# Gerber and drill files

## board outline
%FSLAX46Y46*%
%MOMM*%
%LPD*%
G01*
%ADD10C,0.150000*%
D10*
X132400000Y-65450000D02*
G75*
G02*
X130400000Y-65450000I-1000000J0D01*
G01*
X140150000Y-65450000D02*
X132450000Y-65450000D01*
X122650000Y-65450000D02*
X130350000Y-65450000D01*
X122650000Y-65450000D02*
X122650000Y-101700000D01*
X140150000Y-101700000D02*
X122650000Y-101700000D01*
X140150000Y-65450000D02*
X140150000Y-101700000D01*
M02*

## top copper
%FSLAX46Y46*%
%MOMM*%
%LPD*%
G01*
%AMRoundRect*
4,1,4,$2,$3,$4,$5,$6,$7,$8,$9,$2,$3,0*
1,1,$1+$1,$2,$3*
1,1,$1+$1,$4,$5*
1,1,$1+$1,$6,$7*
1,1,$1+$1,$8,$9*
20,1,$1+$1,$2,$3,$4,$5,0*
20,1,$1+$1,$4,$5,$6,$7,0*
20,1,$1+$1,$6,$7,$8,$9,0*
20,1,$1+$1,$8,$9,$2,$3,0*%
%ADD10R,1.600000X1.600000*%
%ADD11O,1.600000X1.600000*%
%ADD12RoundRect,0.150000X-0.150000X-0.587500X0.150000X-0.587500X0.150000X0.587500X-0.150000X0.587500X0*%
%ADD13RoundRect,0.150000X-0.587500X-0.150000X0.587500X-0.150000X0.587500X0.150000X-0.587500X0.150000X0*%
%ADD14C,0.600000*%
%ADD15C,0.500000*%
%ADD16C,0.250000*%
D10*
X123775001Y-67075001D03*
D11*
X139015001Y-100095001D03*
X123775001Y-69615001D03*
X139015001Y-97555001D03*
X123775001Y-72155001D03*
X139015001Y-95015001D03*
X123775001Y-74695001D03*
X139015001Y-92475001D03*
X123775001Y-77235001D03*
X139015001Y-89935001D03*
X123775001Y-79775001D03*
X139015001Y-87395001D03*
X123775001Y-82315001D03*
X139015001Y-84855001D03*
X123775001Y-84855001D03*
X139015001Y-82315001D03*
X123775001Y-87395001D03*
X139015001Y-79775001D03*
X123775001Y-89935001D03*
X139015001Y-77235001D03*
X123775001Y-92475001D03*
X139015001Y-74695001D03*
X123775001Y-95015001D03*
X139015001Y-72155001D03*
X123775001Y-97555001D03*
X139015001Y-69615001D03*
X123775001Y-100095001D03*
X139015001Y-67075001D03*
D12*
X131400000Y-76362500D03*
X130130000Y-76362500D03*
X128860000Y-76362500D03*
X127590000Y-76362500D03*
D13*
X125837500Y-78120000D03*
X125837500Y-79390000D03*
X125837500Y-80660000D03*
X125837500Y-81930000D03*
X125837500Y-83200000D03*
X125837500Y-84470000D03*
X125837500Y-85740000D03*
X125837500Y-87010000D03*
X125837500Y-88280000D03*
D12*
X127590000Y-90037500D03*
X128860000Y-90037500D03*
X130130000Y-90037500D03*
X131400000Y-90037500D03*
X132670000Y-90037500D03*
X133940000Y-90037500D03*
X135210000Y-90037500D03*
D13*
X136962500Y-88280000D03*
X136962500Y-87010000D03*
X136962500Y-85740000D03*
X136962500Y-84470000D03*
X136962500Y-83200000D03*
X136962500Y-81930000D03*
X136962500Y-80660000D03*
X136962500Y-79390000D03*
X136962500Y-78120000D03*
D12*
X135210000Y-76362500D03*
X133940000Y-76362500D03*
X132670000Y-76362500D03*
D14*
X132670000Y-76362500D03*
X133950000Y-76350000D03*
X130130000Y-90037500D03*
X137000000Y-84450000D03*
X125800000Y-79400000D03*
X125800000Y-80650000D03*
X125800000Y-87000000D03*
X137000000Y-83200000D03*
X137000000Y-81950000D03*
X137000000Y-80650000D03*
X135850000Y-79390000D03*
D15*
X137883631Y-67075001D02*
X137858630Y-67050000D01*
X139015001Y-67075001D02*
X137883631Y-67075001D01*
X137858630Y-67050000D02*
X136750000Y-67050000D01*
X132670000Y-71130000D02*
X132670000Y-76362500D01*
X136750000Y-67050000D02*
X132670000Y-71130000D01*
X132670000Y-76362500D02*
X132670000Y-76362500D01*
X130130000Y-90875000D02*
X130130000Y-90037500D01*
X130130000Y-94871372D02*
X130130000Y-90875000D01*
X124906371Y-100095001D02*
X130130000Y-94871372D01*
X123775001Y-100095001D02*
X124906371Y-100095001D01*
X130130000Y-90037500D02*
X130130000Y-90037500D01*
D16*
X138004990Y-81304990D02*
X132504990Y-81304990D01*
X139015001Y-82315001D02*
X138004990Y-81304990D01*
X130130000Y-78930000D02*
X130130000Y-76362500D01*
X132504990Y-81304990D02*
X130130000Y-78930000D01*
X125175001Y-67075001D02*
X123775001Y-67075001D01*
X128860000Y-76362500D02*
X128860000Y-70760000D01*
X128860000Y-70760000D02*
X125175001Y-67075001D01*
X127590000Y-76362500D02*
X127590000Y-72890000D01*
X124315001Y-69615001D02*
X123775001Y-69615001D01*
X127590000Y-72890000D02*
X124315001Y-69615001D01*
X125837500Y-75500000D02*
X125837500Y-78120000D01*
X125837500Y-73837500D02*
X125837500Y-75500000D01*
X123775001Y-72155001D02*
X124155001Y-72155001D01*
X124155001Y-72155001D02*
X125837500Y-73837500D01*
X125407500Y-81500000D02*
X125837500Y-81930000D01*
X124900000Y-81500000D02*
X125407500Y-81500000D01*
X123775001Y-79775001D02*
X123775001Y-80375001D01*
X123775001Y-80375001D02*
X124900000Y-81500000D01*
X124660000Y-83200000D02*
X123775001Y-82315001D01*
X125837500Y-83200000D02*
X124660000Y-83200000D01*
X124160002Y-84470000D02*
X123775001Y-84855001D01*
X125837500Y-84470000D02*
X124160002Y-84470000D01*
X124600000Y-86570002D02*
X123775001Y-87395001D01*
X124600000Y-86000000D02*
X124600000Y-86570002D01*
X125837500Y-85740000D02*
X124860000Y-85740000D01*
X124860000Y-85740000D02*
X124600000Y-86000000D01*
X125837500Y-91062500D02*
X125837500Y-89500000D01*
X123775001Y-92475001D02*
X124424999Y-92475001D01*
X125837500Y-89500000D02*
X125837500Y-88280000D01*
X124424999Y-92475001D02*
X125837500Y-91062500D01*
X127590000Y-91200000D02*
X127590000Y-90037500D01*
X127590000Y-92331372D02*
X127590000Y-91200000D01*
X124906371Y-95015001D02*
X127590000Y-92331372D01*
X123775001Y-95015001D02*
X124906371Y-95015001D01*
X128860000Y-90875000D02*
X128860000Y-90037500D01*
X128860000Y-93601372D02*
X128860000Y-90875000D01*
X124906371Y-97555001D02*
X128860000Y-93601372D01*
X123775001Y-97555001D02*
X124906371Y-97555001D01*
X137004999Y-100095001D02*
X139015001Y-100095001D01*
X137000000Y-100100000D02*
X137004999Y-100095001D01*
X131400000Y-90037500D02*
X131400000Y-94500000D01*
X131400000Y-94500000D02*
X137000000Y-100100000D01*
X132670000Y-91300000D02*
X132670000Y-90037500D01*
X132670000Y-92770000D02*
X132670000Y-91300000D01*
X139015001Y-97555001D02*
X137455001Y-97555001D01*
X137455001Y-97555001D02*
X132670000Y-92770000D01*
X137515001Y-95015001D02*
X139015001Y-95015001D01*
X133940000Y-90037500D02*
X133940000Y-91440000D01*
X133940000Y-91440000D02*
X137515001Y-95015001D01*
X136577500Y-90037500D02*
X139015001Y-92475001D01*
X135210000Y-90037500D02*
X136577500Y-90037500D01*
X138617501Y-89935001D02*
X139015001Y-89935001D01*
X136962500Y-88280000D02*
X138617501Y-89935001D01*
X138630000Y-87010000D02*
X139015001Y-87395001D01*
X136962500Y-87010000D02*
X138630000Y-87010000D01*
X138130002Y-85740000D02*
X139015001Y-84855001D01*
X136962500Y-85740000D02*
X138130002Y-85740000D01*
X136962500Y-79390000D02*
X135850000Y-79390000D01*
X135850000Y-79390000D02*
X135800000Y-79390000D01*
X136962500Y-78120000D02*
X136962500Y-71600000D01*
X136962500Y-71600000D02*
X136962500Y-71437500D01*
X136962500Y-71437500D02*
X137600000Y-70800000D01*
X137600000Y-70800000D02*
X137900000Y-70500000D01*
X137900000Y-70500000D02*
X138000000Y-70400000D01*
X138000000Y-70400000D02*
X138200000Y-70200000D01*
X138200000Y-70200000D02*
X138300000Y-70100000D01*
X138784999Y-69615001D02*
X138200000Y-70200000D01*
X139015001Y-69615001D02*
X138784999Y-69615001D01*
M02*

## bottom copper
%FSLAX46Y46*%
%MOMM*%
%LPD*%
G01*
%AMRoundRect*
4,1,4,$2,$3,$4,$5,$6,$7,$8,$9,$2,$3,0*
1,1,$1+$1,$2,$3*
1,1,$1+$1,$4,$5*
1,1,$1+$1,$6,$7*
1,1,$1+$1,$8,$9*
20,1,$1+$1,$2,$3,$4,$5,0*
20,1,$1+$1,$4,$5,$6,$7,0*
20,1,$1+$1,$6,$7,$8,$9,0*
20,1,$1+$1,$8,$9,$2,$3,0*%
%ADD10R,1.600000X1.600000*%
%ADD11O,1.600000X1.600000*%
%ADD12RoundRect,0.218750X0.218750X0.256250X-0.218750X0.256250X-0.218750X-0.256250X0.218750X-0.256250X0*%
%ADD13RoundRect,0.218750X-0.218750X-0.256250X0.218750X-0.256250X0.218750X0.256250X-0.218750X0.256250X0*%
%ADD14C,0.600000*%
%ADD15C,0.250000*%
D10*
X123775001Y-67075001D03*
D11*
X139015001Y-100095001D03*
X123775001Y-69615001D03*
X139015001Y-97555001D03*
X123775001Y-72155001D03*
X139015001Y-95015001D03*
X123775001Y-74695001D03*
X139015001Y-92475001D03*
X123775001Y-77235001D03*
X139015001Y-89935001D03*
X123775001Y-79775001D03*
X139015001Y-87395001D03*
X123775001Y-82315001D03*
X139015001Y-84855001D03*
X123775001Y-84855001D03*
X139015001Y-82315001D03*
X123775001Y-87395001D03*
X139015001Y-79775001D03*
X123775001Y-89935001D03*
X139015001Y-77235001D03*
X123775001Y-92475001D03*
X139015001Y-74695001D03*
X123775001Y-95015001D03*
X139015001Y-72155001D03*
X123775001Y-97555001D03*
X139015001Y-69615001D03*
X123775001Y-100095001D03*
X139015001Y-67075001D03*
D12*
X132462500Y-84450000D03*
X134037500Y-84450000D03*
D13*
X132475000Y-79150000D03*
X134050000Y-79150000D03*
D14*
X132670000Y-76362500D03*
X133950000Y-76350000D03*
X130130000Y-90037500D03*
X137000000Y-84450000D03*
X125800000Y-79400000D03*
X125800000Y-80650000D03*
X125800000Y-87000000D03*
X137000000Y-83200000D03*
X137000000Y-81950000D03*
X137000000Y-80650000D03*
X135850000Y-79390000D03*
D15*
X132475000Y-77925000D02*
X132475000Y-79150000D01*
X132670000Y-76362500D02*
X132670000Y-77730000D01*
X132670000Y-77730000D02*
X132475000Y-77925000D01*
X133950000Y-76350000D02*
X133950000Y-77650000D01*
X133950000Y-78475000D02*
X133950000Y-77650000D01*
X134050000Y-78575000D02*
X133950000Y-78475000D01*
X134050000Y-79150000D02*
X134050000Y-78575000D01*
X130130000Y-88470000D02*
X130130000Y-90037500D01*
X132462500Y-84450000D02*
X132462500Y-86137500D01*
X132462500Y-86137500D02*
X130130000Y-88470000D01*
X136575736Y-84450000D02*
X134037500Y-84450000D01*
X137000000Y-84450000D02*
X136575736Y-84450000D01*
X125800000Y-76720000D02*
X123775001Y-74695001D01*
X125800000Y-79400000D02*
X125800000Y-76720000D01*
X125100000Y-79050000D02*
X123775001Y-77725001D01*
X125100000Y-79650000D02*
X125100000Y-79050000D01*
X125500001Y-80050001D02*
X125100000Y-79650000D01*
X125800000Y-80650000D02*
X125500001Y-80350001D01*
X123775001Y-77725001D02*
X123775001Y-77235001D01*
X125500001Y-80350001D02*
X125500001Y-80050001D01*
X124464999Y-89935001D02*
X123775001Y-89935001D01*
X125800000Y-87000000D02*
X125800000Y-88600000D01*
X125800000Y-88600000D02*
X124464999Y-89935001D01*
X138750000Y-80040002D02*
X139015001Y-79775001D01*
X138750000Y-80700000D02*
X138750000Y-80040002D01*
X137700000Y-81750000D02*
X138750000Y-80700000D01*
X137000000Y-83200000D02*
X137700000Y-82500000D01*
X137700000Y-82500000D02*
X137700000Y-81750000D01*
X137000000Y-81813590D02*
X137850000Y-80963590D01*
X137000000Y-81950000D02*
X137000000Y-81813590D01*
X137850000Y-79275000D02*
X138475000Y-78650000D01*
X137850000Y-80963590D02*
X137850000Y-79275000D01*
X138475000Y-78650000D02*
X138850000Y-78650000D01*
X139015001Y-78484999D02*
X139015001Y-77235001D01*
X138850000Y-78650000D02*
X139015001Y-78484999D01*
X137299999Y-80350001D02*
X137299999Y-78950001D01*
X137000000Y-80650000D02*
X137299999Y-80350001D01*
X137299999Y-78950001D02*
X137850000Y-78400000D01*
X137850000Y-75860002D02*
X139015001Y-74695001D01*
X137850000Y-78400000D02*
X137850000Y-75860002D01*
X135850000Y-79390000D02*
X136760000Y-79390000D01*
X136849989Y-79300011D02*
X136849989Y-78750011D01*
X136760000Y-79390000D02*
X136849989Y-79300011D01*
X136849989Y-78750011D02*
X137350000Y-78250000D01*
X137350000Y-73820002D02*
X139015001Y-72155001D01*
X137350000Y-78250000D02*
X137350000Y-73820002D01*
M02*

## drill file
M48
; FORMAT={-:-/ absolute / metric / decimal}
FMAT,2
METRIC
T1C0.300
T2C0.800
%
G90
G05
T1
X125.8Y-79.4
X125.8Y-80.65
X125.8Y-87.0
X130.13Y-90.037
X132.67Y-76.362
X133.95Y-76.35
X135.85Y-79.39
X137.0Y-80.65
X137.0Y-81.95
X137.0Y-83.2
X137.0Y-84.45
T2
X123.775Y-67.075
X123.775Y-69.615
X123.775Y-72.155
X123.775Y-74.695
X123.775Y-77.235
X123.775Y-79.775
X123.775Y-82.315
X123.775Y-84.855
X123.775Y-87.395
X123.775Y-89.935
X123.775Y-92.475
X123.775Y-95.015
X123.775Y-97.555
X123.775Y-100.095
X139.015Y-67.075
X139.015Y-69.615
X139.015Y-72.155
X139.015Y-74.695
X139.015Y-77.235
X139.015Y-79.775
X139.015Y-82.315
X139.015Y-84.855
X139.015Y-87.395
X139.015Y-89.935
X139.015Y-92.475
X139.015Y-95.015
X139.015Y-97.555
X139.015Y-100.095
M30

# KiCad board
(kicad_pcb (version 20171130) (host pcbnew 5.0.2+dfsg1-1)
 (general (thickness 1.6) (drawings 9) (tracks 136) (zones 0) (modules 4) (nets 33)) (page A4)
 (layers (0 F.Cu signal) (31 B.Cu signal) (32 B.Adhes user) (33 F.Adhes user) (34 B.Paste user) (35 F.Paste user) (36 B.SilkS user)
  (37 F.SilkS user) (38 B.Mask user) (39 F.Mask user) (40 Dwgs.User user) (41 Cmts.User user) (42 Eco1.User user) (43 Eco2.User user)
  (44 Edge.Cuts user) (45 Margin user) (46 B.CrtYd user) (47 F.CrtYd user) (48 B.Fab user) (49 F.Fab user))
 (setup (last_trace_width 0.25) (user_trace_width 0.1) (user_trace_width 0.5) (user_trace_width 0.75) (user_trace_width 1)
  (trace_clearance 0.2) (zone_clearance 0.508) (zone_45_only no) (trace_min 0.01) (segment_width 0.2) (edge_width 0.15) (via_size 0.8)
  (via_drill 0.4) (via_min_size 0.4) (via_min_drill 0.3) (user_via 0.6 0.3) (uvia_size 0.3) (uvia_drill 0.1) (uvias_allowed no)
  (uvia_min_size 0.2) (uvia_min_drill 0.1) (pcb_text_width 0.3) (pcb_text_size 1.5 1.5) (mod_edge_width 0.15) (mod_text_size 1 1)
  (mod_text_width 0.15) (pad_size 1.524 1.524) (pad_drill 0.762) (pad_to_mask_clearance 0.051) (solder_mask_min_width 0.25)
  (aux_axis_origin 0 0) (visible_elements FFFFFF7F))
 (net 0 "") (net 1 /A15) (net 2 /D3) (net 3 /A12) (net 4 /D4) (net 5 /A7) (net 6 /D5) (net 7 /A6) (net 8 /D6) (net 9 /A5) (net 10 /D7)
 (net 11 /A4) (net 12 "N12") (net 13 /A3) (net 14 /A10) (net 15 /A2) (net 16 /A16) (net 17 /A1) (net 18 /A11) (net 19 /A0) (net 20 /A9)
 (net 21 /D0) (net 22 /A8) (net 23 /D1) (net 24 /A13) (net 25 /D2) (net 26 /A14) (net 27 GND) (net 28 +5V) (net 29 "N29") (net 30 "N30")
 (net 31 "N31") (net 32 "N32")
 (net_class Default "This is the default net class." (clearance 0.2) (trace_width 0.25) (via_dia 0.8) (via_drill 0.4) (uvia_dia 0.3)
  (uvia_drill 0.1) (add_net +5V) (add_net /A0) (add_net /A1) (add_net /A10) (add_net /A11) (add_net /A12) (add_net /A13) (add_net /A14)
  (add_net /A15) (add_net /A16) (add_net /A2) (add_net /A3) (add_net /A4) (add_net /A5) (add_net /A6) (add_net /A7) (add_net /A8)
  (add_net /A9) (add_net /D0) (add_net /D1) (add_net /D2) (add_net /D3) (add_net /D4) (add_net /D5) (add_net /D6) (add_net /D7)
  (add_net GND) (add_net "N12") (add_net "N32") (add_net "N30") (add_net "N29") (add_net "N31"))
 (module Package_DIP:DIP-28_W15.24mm (layer F.Cu) (at 123.775001 67.075001)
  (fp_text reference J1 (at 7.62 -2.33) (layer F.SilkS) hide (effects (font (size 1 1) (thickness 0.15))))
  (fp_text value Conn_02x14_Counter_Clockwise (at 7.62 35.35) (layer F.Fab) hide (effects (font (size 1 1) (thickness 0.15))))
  (pad 1 thru_hole rect (at 0 0) (size 1.6 1.6) (drill 0.8) (layers *.Cu *.Mask) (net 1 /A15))
  (pad 15 thru_hole oval (at 15.24 33.02) (size 1.6 1.6) (drill 0.8) (layers *.Cu *.Mask) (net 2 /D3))
  (pad 2 thru_hole oval (at 0 2.54) (size 1.6 1.6) (drill 0.8) (layers *.Cu *.Mask) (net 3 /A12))
  (pad 16 thru_hole oval (at 15.24 30.48) (size 1.6 1.6) (drill 0.8) (layers *.Cu *.Mask) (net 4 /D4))
  (pad 3 thru_hole oval (at 0 5.08) (size 1.6 1.6) (drill 0.8) (layers *.Cu *.Mask) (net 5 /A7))
  (pad 17 thru_hole oval (at 15.24 27.94) (size 1.6 1.6) (drill 0.8) (layers *.Cu *.Mask) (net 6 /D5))
  (pad 4 thru_hole oval (at 0 7.62) (size 1.6 1.6) (drill 0.8) (layers *.Cu *.Mask) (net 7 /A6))
  (pad 18 thru_hole oval (at 15.24 25.4) (size 1.6 1.6) (drill 0.8) (layers *.Cu *.Mask) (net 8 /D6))
  (pad 5 thru_hole oval (at 0 10.16) (size 1.6 1.6) (drill 0.8) (layers *.Cu *.Mask) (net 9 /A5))
  (pad 19 thru_hole oval (at 15.24 22.86) (size 1.6 1.6) (drill 0.8) (layers *.Cu *.Mask) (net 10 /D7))
  (pad 6 thru_hole oval (at 0 12.7) (size 1.6 1.6) (drill 0.8) (layers *.Cu *.Mask) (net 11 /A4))
  (pad 20 thru_hole oval (at 15.24 20.32) (size 1.6 1.6) (drill 0.8) (layers *.Cu *.Mask) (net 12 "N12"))
  (pad 7 thru_hole oval (at 0 15.24) (size 1.6 1.6) (drill 0.8) (layers *.Cu *.Mask) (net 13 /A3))
  (pad 21 thru_hole oval (at 15.24 17.78) (size 1.6 1.6) (drill 0.8) (layers *.Cu *.Mask) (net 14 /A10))
  (pad 8 thru_hole oval (at 0 17.78) (size 1.6 1.6) (drill 0.8) (layers *.Cu *.Mask) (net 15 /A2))
  (pad 22 thru_hole oval (at 15.24 15.24) (size 1.6 1.6) (drill 0.8) (layers *.Cu *.Mask) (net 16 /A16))
  (pad 9 thru_hole oval (at 0 20.32) (size 1.6 1.6) (drill 0.8) (layers *.Cu *.Mask) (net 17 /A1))
  (pad 23 thru_hole oval (at 15.24 12.7) (size 1.6 1.6) (drill 0.8) (layers *.Cu *.Mask) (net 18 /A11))
  (pad 10 thru_hole oval (at 0 22.86) (size 1.6 1.6) (drill 0.8) (layers *.Cu *.Mask) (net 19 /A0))
  (pad 24 thru_hole oval (at 15.24 10.16) (size 1.6 1.6) (drill 0.8) (layers *.Cu *.Mask) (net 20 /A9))
  (pad 11 thru_hole oval (at 0 25.4) (size 1.6 1.6) (drill 0.8) (layers *.Cu *.Mask) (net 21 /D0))
  (pad 25 thru_hole oval (at 15.24 7.62) (size 1.6 1.6) (drill 0.8) (layers *.Cu *.Mask) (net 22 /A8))
  (pad 12 thru_hole oval (at 0 27.94) (size 1.6 1.6) (drill 0.8) (layers *.Cu *.Mask) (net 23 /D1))
  (pad 26 thru_hole oval (at 15.24 5.08) (size 1.6 1.6) (drill 0.8) (layers *.Cu *.Mask) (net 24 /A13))
  (pad 13 thru_hole oval (at 0 30.48) (size 1.6 1.6) (drill 0.8) (layers *.Cu *.Mask) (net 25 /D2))
  (pad 27 thru_hole oval (at 15.24 2.54) (size 1.6 1.6) (drill 0.8) (layers *.Cu *.Mask) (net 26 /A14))
  (pad 14 thru_hole oval (at 0 33.02) (size 1.6 1.6) (drill 0.8) (layers *.Cu *.Mask) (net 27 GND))
  (pad 28 thru_hole oval (at 15.24 0) (size 1.6 1.6) (drill 0.8) (layers *.Cu *.Mask) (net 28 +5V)))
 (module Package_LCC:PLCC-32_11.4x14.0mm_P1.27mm (layer F.Cu) (at 131.4 83.2)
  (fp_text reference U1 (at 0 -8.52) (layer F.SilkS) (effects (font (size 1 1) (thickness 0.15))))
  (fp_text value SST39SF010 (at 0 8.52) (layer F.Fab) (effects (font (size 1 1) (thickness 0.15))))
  (pad 1 smd roundrect (at 0 -6.8375) (size 0.6 1.475) (layers F.Cu F.Paste F.Mask) (roundrect_rratio 0.25) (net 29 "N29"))
  (pad 2 smd roundrect (at -1.27 -6.8375) (size 0.6 1.475) (layers F.Cu F.Paste F.Mask) (roundrect_rratio 0.25) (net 16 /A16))
  (pad 3 smd roundrect (at -2.54 -6.8375) (size 0.6 1.475) (layers F.Cu F.Paste F.Mask) (roundrect_rratio 0.25) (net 1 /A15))
  (pad 4 smd roundrect (at -3.81 -6.8375) (size 0.6 1.475) (layers F.Cu F.Paste F.Mask) (roundrect_rratio 0.25) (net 3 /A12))
  (pad 5 smd roundrect (at -5.5625 -5.08) (size 1.475 0.6) (layers F.Cu F.Paste F.Mask) (roundrect_rratio 0.25) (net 5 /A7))
  (pad 6 smd roundrect (at -5.5625 -3.81) (size 1.475 0.6) (layers F.Cu F.Paste F.Mask) (roundrect_rratio 0.25) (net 7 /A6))
  (pad 7 smd roundrect (at -5.5625 -2.54) (size 1.475 0.6) (layers F.Cu F.Paste F.Mask) (roundrect_rratio 0.25) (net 9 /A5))
  (pad 8 smd roundrect (at -5.5625 -1.27) (size 1.475 0.6) (layers F.Cu F.Paste F.Mask) (roundrect_rratio 0.25) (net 11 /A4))
  (pad 9 smd roundrect (at -5.5625 0) (size 1.475 0.6) (layers F.Cu F.Paste F.Mask) (roundrect_rratio 0.25) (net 13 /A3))
  (pad 10 smd roundrect (at -5.5625 1.27) (size 1.475 0.6) (layers F.Cu F.Paste F.Mask) (roundrect_rratio 0.25) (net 15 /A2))
  (pad 11 smd roundrect (at -5.5625 2.54) (size 1.475 0.6) (layers F.Cu F.Paste F.Mask) (roundrect_rratio 0.25) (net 17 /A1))
  (pad 12 smd roundrect (at -5.5625 3.81) (size 1.475 0.6) (layers F.Cu F.Paste F.Mask) (roundrect_rratio 0.25) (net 19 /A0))
  (pad 13 smd roundrect (at -5.5625 5.08) (size 1.475 0.6) (layers F.Cu F.Paste F.Mask) (roundrect_rratio 0.25) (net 21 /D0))
  (pad 14 smd roundrect (at -3.81 6.8375) (size 0.6 1.475) (layers F.Cu F.Paste F.Mask) (roundrect_rratio 0.25) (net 23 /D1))
  (pad 15 smd roundrect (at -2.54 6.8375) (size 0.6 1.475) (layers F.Cu F.Paste F.Mask) (roundrect_rratio 0.25) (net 25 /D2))
  (pad 16 smd roundrect (at -1.27 6.8375) (size 0.6 1.475) (layers F.Cu F.Paste F.Mask) (roundrect_rratio 0.25) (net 27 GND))
  (pad 17 smd roundrect (at 0 6.8375) (size 0.6 1.475) (layers F.Cu F.Paste F.Mask) (roundrect_rratio 0.25) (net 2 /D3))
  (pad 18 smd roundrect (at 1.27 6.8375) (size 0.6 1.475) (layers F.Cu F.Paste F.Mask) (roundrect_rratio 0.25) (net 4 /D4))
  (pad 19 smd roundrect (at 2.54 6.8375) (size 0.6 1.475) (layers F.Cu F.Paste F.Mask) (roundrect_rratio 0.25) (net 6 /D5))
  (pad 20 smd roundrect (at 3.81 6.8375) (size 0.6 1.475) (layers F.Cu F.Paste F.Mask) (roundrect_rratio 0.25) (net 8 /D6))
  (pad 21 smd roundrect (at 5.5625 5.08) (size 1.475 0.6) (layers F.Cu F.Paste F.Mask) (roundrect_rratio 0.25) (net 10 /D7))
  (pad 22 smd roundrect (at 5.5625 3.81) (size 1.475 0.6) (layers F.Cu F.Paste F.Mask) (roundrect_rratio 0.25) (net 12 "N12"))
  (pad 23 smd roundrect (at 5.5625 2.54) (size 1.475 0.6) (layers F.Cu F.Paste F.Mask) (roundrect_rratio 0.25) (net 14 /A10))
  (pad 24 smd roundrect (at 5.5625 1.27) (size 1.475 0.6) (layers F.Cu F.Paste F.Mask) (roundrect_rratio 0.25) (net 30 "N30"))
  (pad 25 smd roundrect (at 5.5625 0) (size 1.475 0.6) (layers F.Cu F.Paste F.Mask) (roundrect_rratio 0.25) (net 18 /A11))
  (pad 26 smd roundrect (at 5.5625 -1.27) (size 1.475 0.6) (layers F.Cu F.Paste F.Mask) (roundrect_rratio 0.25) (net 20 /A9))
  (pad 27 smd roundrect (at 5.5625 -2.54) (size 1.475 0.6) (layers F.Cu F.Paste F.Mask) (roundrect_rratio 0.25) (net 22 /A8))
  (pad 28 smd roundrect (at 5.5625 -3.81) (size 1.475 0.6) (layers F.Cu F.Paste F.Mask) (roundrect_rratio 0.25) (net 24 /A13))
  (pad 29 smd roundrect (at 5.5625 -5.08) (size 1.475 0.6) (layers F.Cu F.Paste F.Mask) (roundrect_rratio 0.25) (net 26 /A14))
  (pad 30 smd roundrect (at 3.81 -6.8375) (size 0.6 1.475) (layers F.Cu F.Paste F.Mask) (roundrect_rratio 0.25) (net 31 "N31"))
  (pad 31 smd roundrect (at 2.54 -6.8375) (size 0.6 1.475) (layers F.Cu F.Paste F.Mask) (roundrect_rratio 0.25) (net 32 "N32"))
  (pad 32 smd roundrect (at 1.27 -6.8375) (size 0.6 1.475) (layers F.Cu F.Paste F.Mask) (roundrect_rratio 0.25) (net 28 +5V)))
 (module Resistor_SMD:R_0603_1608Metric (layer B.Cu) (at 133.25 84.45 180)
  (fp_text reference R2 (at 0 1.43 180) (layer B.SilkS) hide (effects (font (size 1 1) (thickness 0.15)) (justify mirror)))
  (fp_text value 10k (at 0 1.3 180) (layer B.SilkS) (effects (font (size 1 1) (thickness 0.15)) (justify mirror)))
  (pad 2 smd roundrect (at 0.7875 0 180) (size 0.875 0.95) (layers B.Cu B.Paste B.Mask) (roundrect_rratio 0.25) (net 27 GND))
  (pad 1 smd roundrect (at -0.7875 0 180) (size 0.875 0.95) (layers B.Cu B.Paste B.Mask) (roundrect_rratio 0.25) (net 30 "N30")))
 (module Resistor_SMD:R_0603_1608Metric (layer B.Cu) (at 133.2625 79.15)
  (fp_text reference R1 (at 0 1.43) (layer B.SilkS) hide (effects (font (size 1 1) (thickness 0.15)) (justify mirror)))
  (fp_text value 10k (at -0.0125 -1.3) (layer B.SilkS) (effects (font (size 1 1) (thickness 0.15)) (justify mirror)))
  (pad 1 smd roundrect (at -0.7875 0) (size 0.875 0.95) (layers B.Cu B.Paste B.Mask) (roundrect_rratio 0.25) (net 28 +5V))
  (pad 2 smd roundrect (at 0.7875 0) (size 0.875 0.95) (layers B.Cu B.Paste B.Mask) (roundrect_rratio 0.25) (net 32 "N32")))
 (gr_arc (start 131.4 65.45) (end 130.4 65.45) (angle -180) (layer Edge.Cuts) (width 0.15))
 (gr_line (start 140.15 65.45) (end 132.45 65.45) (layer Edge.Cuts) (width 0.15))
 (gr_line (start 122.65 65.45) (end 130.35 65.45) (layer Edge.Cuts) (width 0.15))
 (gr_line (start 122.65 65.45) (end 122.65 101.7) (layer Edge.Cuts) (width 0.15))
 (gr_line (start 140.15 101.7) (end 122.65 101.7) (layer Edge.Cuts) (width 0.15))
 (gr_line (start 140.15 65.45) (end 140.15 101.7) (layer Edge.Cuts) (width 0.15))
 (segment (start 137.883631 67.075001) (end 137.85863 67.05) (width 0.5) (layer F.Cu) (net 28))
 (segment (start 139.015001 67.075001) (end 137.883631 67.075001) (width 0.5) (layer F.Cu) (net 28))
 (segment (start 137.85863 67.05) (end 136.75 67.05) (width 0.5) (layer F.Cu) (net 28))
 (segment (start 132.67 71.13) (end 132.67 76.3625) (width 0.5) (layer F.Cu) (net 28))
 (segment (start 136.75 67.05) (end 132.67 71.13) (width 0.5) (layer F.Cu) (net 28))
 (segment (start 132.67 76.3625) (end 132.67 76.3625) (width 0.5) (layer F.Cu) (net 28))
 (via (at 132.67 76.3625) (size 0.6) (drill 0.3) (layers F.Cu B.Cu) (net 28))
 (segment (start 132.475 77.925) (end 132.475 79.15) (width 0.25) (layer B.Cu) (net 28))
 (segment (start 132.67 76.3625) (end 132.67 77.73) (width 0.25) (layer B.Cu) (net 28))
 (segment (start 132.67 77.73) (end 132.475 77.925) (width 0.25) (layer B.Cu) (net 28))
 (via (at 133.95 76.35) (size 0.6) (drill 0.3) (layers F.Cu B.Cu) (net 32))
 (segment (start 133.95 76.35) (end 133.95 77.65) (width 0.25) (layer B.Cu) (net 32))
 (segment (start 133.95 78.475) (end 133.95 77.65) (width 0.25) (layer B.Cu) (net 32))
 (segment (start 134.05 78.575) (end 133.95 78.475) (width 0.25) (layer B.Cu) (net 32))
 (segment (start 134.05 79.15) (end 134.05 78.575) (width 0.25) (layer B.Cu) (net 32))
 (segment (start 130.13 90.875) (end 130.13 90.0375) (width 0.5) (layer F.Cu) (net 27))
 (segment (start 130.13 94.871372) (end 130.13 90.875) (width 0.5) (layer F.Cu) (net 27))
 (segment (start 124.906371 100.095001) (end 130.13 94.871372) (width 0.5) (layer F.Cu) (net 27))
 (segment (start 123.775001 100.095001) (end 124.906371 100.095001) (width 0.5) (layer F.Cu) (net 27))
 (segment (start 130.13 90.0375) (end 130.13 90.0375) (width 0.5) (layer F.Cu) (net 27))
 (via (at 130.13 90.0375) (size 0.6) (drill 0.3) (layers F.Cu B.Cu) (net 27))
 (segment (start 130.13 88.47) (end 130.13 90.0375) (width 0.25) (layer B.Cu) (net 27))
 (segment (start 132.4625 84.45) (end 132.4625 86.1375) (width 0.25) (layer B.Cu) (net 27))
 (segment (start 132.4625 86.1375) (end 130.13 88.47) (width 0.25) (layer B.Cu) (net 27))
 (via (at 137 84.45) (size 0.6) (drill 0.3) (layers F.Cu B.Cu) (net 30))
 (segment (start 136.575736 84.45) (end 134.0375 84.45) (width 0.25) (layer B.Cu) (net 30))
 (segment (start 137 84.45) (end 136.575736 84.45) (width 0.25) (layer B.Cu) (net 30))
 (segment (start 138.00499 81.30499) (end 132.50499 81.30499) (width 0.25) (layer F.Cu) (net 16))
 (segment (start 139.015001 82.315001) (end 138.00499 81.30499) (width 0.25) (layer F.Cu) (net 16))
 (segment (start 130.13 78.93) (end 130.13 76.3625) (width 0.25) (layer F.Cu) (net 16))
 (segment (start 132.50499 81.30499) (end 130.13 78.93) (width 0.25) (layer F.Cu) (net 16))
 (segment (start 125.175001 67.075001) (end 123.775001 67.075001) (width 0.25) (layer F.Cu) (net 1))
 (segment (start 128.86 76.3625) (end 128.86 70.76) (width 0.25) (layer F.Cu) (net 1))
 (segment (start 128.86 70.76) (end 125.175001 67.075001) (width 0.25) (layer F.Cu) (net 1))
 (segment (start 127.59 76.3625) (end 127.59 72.89) (width 0.25) (layer F.Cu) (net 3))
 (segment (start 124.315001 69.615001) (end 123.775001 69.615001) (width 0.25) (layer F.Cu) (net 3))
 (segment (start 127.59 72.89) (end 124.315001 69.615001) (width 0.25) (layer F.Cu) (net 3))
 (segment (start 125.8375 75.5) (end 125.8375 78.12) (width 0.25) (layer F.Cu) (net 5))
 (segment (start 125.8375 73.8375) (end 125.8375 75.5) (width 0.25) (layer F.Cu) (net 5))
 (segment (start 123.775001 72.155001) (end 124.155001 72.155001) (width 0.25) (layer F.Cu) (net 5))
 (segment (start 124.155001 72.155001) (end 125.8375 73.8375) (width 0.25) (layer F.Cu) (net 5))
 (via (at 125.8 79.4) (size 0.6) (drill 0.3) (layers F.Cu B.Cu) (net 7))
 (segment (start 125.8 76.72) (end 123.775001 74.695001) (width 0.25) (layer B.Cu) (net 7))
 (segment (start 125.8 79.4) (end 125.8 76.72) (width 0.25) (layer B.Cu) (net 7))
 (via (at 125.8 80.65) (size 0.6) (drill 0.3) (layers F.Cu B.Cu) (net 9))
 (segment (start 125.1 79.05) (end 123.775001 77.725001) (width 0.25) (layer B.Cu) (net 9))
 (segment (start 125.1 79.65) (end 125.1 79.05) (width 0.25) (layer B.Cu) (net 9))
 (segment (start 125.500001 80.050001) (end 125.1 79.65) (width 0.25) (layer B.Cu) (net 9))
 (segment (start 125.8 80.65) (end 125.500001 80.350001) (width 0.25) (layer B.Cu) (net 9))
 (segment (start 123.775001 77.725001) (end 123.775001 77.235001) (width 0.25) (layer B.Cu) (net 9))
 (segment (start 125.500001 80.350001) (end 125.500001 80.050001) (width 0.25) (layer B.Cu) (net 9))
 (segment (start 125.4075 81.5) (end 125.8375 81.93) (width 0.25) (layer F.Cu) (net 11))
 (segment (start 124.9 81.5) (end 125.4075 81.5) (width 0.25) (layer F.Cu) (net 11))
 (segment (start 123.775001 79.775001) (end 123.775001 80.375001) (width 0.25) (layer F.Cu) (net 11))
 (segment (start 123.775001 80.375001) (end 124.9 81.5) (width 0.25) (layer F.Cu) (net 11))
 (segment (start 124.66 83.2) (end 123.775001 82.315001) (width 0.25) (layer F.Cu) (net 13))
 (segment (start 125.8375 83.2) (end 124.66 83.2) (width 0.25) (layer F.Cu) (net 13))
 (segment (start 124.160002 84.47) (end 123.775001 84.855001) (width 0.25) (layer F.Cu) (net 15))
 (segment (start 125.8375 84.47) (end 124.160002 84.47) (width 0.25) (layer F.Cu) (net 15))
 (segment (start 124.6 86.570002) (end 123.775001 87.395001) (width 0.25) (layer F.Cu) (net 17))
 (segment (start 124.6 86) (end 124.6 86.570002) (width 0.25) (layer F.Cu) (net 17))
 (segment (start 125.8375 85.74) (end 124.86 85.74) (width 0.25) (layer F.Cu) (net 17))
 (segment (start 124.86 85.74) (end 124.6 86) (width 0.25) (layer F.Cu) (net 17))
 (via (at 125.8 87) (size 0.6) (drill 0.3) (layers F.Cu B.Cu) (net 19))
 (segment (start 124.464999 89.935001) (end 123.775001 89.935001) (width 0.25) (layer B.Cu) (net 19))
 (segment (start 125.8 87) (end 125.8 88.6) (width 0.25) (layer B.Cu) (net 19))
 (segment (start 125.8 88.6) (end 124.464999 89.935001) (width 0.25) (layer B.Cu) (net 19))
 (segment (start 125.8375 91.0625) (end 125.8375 89.5) (width 0.25) (layer F.Cu) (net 21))
 (segment (start 123.775001 92.475001) (end 124.424999 92.475001) (width 0.25) (layer F.Cu) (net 21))
 (segment (start 125.8375 89.5) (end 125.8375 88.28) (width 0.25) (layer F.Cu) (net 21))
 (segment (start 124.424999 92.475001) (end 125.8375 91.0625) (width 0.25) (layer F.Cu) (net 21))
 (segment (start 127.59 91.2) (end 127.59 90.0375) (width 0.25) (layer F.Cu) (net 23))
 (segment (start 127.59 92.331372) (end 127.59 91.2) (width 0.25) (layer F.Cu) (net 23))
 (segment (start 124.906371 95.015001) (end 127.59 92.331372) (width 0.25) (layer F.Cu) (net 23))
 (segment (start 123.775001 95.015001) (end 124.906371 95.015001) (width 0.25) (layer F.Cu) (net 23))
 (segment (start 128.86 90.875) (end 128.86 90.0375) (width 0.25) (layer F.Cu) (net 25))
 (segment (start 128.86 93.601372) (end 128.86 90.875) (width 0.25) (layer F.Cu) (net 25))
 (segment (start 124.906371 97.555001) (end 128.86 93.601372) (width 0.25) (layer F.Cu) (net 25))
 (segment (start 123.775001 97.555001) (end 124.906371 97.555001) (width 0.25) (layer F.Cu) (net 25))
 (segment (start 137.004999 100.095001) (end 139.015001 100.095001) (width 0.25) (layer F.Cu) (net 2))
 (segment (start 137 100.1) (end 137.004999 100.095001) (width 0.25) (layer F.Cu) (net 2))
 (segment (start 131.4 90.0375) (end 131.4 94.5) (width 0.25) (layer F.Cu) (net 2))
 (segment (start 131.4 94.5) (end 137 100.1) (width 0.25) (layer F.Cu) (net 2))
 (segment (start 132.67 91.3) (end 132.67 90.0375) (width 0.25) (layer F.Cu) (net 4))
 (segment (start 132.67 92.77) (end 132.67 91.3) (width 0.25) (layer F.Cu) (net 4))
 (segment (start 139.015001 97.555001) (end 137.455001 97.555001) (width 0.25) (layer F.Cu) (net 4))
 (segment (start 137.455001 97.555001) (end 132.67 92.77) (width 0.25) (layer F.Cu) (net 4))
 (segment (start 137.515001 95.015001) (end 139.015001 95.015001) (width 0.25) (layer F.Cu) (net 6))
 (segment (start 133.94 90.0375) (end 133.94 91.44) (width 0.25) (layer F.Cu) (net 6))
 (segment (start 133.94 91.44) (end 137.515001 95.015001) (width 0.25) (layer F.Cu) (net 6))
 (segment (start 136.5775 90.0375) (end 139.015001 92.475001) (width 0.25) (layer F.Cu) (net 8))
 (segment (start 135.21 90.0375) (end 136.5775 90.0375) (width 0.25) (layer F.Cu) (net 8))
 (segment (start 138.617501 89.935001) (end 139.015001 89.935001) (width 0.25) (layer F.Cu) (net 10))
 (segment (start 136.9625 88.28) (end 138.617501 89.935001) (width 0.25) (layer F.Cu) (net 10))
 (segment (start 138.63 87.01) (end 139.015001 87.395001) (width 0.25) (layer F.Cu) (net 12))
 (segment (start 136.9625 87.01) (end 138.63 87.01) (width 0.25) (layer F.Cu) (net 12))
 (segment (start 138.130002 85.74) (end 139.015001 84.855001) (width 0.25) (layer F.Cu) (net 14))
 (segment (start 136.9625 85.74) (end 138.130002 85.74) (width 0.25) (layer F.Cu) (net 14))
 (via (at 137 83.2) (size 0.6) (drill 0.3) (layers F.Cu B.Cu) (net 18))
 (segment (start 138.75 80.040002) (end 139.015001 79.775001) (width 0.25) (layer B.Cu) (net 18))
 (segment (start 138.75 80.7) (end 138.75 80.040002) (width 0.25) (layer B.Cu) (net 18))
 (segment (start 137.7 81.75) (end 138.75 80.7) (width 0.25) (layer B.Cu) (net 18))
 (segment (start 137 83.2) (end 137.7 82.5) (width 0.25) (layer B.Cu) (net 18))
 (segment (start 137.7 82.5) (end 137.7 81.75) (width 0.25) (layer B.Cu) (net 18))
 (via (at 137 81.95) (size 0.6) (drill 0.3) (layers F.Cu B.Cu) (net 20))
 (segment (start 137 81.81359) (end 137.85 80.96359) (width 0.25) (layer B.Cu) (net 20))
 (segment (start 137 81.95) (end 137 81.81359) (width 0.25) (layer B.Cu) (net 20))
 (segment (start 137.85 79.275) (end 138.475 78.65) (width 0.25) (layer B.Cu) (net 20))
 (segment (start 137.85 80.96359) (end 137.85 79.275) (width 0.25) (layer B.Cu) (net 20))
 (segment (start 138.475 78.65) (end 138.85 78.65) (width 0.25) (layer B.Cu) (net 20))
 (segment (start 139.015001 78.484999) (end 139.015001 77.235001) (width 0.25) (layer B.Cu) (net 20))
 (segment (start 138.85 78.65) (end 139.015001 78.484999) (width 0.25) (layer B.Cu) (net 20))
 (via (at 137 80.65) (size 0.6) (drill 0.3) (layers F.Cu B.Cu) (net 22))
 (segment (start 137.299999 80.350001) (end 137.299999 78.950001) (width 0.25) (layer B.Cu) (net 22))
 (segment (start 137 80.65) (end 137.299999 80.350001) (width 0.25) (layer B.Cu) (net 22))
 (segment (start 137.299999 78.950001) (end 137.85 78.4) (width 0.25) (layer B.Cu) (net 22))
 (segment (start 137.85 75.860002) (end 139.015001 74.695001) (width 0.25) (layer B.Cu) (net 22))
 (segment (start 137.85 78.4) (end 137.85 75.860002) (width 0.25) (layer B.Cu) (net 22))
 (segment (start 136.9625 79.39) (end 135.85 79.39) (width 0.25) (layer F.Cu) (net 24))
 (segment (start 135.85 79.39) (end 135.8 79.39) (width 0.25) (layer F.Cu) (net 24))
 (via (at 135.85 79.39) (size 0.6) (drill 0.3) (layers F.Cu B.Cu) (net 24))
 (segment (start 135.85 79.39) (end 136.76 79.39) (width 0.25) (layer B.Cu) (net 24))
 (segment (start 136.849989 79.300011) (end 136.849989 78.750011) (width 0.25) (layer B.Cu) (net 24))
 (segment (start 136.76 79.39) (end 136.849989 79.300011) (width 0.25) (layer B.Cu) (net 24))
 (segment (start 136.849989 78.750011) (end 137.35 78.25) (width 0.25) (layer B.Cu) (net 24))
 (segment (start 137.35 73.820002) (end 139.015001 72.155001) (width 0.25) (layer B.Cu) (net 24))
 (segment (start 137.35 78.25) (end 137.35 73.820002) (width 0.25) (layer B.Cu) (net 24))
 (segment (start 136.9625 78.12) (end 136.9625 71.6) (width 0.25) (layer F.Cu) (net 26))
 (segment (start 136.9625 71.6) (end 136.9625 71.4375) (width 0.25) (layer F.Cu) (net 26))
 (segment (start 136.9625 71.4375) (end 137.6 70.8) (width 0.25) (layer F.Cu) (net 26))
 (segment (start 137.6 70.8) (end 137.9 70.5) (width 0.25) (layer F.Cu) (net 26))
 (segment (start 137.9 70.5) (end 138 70.4) (width 0.25) (layer F.Cu) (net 26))
 (segment (start 138 70.4) (end 138.2 70.2) (width 0.25) (layer F.Cu) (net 26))
 (segment (start 138.2 70.2) (end 138.3 70.1) (width 0.25) (layer F.Cu) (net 26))
 (segment (start 138.784999 69.615001) (end 138.2 70.2) (width 0.25) (layer F.Cu) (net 26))
 (segment (start 139.015001 69.615001) (end 138.784999 69.615001) (width 0.25) (layer F.Cu) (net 26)))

